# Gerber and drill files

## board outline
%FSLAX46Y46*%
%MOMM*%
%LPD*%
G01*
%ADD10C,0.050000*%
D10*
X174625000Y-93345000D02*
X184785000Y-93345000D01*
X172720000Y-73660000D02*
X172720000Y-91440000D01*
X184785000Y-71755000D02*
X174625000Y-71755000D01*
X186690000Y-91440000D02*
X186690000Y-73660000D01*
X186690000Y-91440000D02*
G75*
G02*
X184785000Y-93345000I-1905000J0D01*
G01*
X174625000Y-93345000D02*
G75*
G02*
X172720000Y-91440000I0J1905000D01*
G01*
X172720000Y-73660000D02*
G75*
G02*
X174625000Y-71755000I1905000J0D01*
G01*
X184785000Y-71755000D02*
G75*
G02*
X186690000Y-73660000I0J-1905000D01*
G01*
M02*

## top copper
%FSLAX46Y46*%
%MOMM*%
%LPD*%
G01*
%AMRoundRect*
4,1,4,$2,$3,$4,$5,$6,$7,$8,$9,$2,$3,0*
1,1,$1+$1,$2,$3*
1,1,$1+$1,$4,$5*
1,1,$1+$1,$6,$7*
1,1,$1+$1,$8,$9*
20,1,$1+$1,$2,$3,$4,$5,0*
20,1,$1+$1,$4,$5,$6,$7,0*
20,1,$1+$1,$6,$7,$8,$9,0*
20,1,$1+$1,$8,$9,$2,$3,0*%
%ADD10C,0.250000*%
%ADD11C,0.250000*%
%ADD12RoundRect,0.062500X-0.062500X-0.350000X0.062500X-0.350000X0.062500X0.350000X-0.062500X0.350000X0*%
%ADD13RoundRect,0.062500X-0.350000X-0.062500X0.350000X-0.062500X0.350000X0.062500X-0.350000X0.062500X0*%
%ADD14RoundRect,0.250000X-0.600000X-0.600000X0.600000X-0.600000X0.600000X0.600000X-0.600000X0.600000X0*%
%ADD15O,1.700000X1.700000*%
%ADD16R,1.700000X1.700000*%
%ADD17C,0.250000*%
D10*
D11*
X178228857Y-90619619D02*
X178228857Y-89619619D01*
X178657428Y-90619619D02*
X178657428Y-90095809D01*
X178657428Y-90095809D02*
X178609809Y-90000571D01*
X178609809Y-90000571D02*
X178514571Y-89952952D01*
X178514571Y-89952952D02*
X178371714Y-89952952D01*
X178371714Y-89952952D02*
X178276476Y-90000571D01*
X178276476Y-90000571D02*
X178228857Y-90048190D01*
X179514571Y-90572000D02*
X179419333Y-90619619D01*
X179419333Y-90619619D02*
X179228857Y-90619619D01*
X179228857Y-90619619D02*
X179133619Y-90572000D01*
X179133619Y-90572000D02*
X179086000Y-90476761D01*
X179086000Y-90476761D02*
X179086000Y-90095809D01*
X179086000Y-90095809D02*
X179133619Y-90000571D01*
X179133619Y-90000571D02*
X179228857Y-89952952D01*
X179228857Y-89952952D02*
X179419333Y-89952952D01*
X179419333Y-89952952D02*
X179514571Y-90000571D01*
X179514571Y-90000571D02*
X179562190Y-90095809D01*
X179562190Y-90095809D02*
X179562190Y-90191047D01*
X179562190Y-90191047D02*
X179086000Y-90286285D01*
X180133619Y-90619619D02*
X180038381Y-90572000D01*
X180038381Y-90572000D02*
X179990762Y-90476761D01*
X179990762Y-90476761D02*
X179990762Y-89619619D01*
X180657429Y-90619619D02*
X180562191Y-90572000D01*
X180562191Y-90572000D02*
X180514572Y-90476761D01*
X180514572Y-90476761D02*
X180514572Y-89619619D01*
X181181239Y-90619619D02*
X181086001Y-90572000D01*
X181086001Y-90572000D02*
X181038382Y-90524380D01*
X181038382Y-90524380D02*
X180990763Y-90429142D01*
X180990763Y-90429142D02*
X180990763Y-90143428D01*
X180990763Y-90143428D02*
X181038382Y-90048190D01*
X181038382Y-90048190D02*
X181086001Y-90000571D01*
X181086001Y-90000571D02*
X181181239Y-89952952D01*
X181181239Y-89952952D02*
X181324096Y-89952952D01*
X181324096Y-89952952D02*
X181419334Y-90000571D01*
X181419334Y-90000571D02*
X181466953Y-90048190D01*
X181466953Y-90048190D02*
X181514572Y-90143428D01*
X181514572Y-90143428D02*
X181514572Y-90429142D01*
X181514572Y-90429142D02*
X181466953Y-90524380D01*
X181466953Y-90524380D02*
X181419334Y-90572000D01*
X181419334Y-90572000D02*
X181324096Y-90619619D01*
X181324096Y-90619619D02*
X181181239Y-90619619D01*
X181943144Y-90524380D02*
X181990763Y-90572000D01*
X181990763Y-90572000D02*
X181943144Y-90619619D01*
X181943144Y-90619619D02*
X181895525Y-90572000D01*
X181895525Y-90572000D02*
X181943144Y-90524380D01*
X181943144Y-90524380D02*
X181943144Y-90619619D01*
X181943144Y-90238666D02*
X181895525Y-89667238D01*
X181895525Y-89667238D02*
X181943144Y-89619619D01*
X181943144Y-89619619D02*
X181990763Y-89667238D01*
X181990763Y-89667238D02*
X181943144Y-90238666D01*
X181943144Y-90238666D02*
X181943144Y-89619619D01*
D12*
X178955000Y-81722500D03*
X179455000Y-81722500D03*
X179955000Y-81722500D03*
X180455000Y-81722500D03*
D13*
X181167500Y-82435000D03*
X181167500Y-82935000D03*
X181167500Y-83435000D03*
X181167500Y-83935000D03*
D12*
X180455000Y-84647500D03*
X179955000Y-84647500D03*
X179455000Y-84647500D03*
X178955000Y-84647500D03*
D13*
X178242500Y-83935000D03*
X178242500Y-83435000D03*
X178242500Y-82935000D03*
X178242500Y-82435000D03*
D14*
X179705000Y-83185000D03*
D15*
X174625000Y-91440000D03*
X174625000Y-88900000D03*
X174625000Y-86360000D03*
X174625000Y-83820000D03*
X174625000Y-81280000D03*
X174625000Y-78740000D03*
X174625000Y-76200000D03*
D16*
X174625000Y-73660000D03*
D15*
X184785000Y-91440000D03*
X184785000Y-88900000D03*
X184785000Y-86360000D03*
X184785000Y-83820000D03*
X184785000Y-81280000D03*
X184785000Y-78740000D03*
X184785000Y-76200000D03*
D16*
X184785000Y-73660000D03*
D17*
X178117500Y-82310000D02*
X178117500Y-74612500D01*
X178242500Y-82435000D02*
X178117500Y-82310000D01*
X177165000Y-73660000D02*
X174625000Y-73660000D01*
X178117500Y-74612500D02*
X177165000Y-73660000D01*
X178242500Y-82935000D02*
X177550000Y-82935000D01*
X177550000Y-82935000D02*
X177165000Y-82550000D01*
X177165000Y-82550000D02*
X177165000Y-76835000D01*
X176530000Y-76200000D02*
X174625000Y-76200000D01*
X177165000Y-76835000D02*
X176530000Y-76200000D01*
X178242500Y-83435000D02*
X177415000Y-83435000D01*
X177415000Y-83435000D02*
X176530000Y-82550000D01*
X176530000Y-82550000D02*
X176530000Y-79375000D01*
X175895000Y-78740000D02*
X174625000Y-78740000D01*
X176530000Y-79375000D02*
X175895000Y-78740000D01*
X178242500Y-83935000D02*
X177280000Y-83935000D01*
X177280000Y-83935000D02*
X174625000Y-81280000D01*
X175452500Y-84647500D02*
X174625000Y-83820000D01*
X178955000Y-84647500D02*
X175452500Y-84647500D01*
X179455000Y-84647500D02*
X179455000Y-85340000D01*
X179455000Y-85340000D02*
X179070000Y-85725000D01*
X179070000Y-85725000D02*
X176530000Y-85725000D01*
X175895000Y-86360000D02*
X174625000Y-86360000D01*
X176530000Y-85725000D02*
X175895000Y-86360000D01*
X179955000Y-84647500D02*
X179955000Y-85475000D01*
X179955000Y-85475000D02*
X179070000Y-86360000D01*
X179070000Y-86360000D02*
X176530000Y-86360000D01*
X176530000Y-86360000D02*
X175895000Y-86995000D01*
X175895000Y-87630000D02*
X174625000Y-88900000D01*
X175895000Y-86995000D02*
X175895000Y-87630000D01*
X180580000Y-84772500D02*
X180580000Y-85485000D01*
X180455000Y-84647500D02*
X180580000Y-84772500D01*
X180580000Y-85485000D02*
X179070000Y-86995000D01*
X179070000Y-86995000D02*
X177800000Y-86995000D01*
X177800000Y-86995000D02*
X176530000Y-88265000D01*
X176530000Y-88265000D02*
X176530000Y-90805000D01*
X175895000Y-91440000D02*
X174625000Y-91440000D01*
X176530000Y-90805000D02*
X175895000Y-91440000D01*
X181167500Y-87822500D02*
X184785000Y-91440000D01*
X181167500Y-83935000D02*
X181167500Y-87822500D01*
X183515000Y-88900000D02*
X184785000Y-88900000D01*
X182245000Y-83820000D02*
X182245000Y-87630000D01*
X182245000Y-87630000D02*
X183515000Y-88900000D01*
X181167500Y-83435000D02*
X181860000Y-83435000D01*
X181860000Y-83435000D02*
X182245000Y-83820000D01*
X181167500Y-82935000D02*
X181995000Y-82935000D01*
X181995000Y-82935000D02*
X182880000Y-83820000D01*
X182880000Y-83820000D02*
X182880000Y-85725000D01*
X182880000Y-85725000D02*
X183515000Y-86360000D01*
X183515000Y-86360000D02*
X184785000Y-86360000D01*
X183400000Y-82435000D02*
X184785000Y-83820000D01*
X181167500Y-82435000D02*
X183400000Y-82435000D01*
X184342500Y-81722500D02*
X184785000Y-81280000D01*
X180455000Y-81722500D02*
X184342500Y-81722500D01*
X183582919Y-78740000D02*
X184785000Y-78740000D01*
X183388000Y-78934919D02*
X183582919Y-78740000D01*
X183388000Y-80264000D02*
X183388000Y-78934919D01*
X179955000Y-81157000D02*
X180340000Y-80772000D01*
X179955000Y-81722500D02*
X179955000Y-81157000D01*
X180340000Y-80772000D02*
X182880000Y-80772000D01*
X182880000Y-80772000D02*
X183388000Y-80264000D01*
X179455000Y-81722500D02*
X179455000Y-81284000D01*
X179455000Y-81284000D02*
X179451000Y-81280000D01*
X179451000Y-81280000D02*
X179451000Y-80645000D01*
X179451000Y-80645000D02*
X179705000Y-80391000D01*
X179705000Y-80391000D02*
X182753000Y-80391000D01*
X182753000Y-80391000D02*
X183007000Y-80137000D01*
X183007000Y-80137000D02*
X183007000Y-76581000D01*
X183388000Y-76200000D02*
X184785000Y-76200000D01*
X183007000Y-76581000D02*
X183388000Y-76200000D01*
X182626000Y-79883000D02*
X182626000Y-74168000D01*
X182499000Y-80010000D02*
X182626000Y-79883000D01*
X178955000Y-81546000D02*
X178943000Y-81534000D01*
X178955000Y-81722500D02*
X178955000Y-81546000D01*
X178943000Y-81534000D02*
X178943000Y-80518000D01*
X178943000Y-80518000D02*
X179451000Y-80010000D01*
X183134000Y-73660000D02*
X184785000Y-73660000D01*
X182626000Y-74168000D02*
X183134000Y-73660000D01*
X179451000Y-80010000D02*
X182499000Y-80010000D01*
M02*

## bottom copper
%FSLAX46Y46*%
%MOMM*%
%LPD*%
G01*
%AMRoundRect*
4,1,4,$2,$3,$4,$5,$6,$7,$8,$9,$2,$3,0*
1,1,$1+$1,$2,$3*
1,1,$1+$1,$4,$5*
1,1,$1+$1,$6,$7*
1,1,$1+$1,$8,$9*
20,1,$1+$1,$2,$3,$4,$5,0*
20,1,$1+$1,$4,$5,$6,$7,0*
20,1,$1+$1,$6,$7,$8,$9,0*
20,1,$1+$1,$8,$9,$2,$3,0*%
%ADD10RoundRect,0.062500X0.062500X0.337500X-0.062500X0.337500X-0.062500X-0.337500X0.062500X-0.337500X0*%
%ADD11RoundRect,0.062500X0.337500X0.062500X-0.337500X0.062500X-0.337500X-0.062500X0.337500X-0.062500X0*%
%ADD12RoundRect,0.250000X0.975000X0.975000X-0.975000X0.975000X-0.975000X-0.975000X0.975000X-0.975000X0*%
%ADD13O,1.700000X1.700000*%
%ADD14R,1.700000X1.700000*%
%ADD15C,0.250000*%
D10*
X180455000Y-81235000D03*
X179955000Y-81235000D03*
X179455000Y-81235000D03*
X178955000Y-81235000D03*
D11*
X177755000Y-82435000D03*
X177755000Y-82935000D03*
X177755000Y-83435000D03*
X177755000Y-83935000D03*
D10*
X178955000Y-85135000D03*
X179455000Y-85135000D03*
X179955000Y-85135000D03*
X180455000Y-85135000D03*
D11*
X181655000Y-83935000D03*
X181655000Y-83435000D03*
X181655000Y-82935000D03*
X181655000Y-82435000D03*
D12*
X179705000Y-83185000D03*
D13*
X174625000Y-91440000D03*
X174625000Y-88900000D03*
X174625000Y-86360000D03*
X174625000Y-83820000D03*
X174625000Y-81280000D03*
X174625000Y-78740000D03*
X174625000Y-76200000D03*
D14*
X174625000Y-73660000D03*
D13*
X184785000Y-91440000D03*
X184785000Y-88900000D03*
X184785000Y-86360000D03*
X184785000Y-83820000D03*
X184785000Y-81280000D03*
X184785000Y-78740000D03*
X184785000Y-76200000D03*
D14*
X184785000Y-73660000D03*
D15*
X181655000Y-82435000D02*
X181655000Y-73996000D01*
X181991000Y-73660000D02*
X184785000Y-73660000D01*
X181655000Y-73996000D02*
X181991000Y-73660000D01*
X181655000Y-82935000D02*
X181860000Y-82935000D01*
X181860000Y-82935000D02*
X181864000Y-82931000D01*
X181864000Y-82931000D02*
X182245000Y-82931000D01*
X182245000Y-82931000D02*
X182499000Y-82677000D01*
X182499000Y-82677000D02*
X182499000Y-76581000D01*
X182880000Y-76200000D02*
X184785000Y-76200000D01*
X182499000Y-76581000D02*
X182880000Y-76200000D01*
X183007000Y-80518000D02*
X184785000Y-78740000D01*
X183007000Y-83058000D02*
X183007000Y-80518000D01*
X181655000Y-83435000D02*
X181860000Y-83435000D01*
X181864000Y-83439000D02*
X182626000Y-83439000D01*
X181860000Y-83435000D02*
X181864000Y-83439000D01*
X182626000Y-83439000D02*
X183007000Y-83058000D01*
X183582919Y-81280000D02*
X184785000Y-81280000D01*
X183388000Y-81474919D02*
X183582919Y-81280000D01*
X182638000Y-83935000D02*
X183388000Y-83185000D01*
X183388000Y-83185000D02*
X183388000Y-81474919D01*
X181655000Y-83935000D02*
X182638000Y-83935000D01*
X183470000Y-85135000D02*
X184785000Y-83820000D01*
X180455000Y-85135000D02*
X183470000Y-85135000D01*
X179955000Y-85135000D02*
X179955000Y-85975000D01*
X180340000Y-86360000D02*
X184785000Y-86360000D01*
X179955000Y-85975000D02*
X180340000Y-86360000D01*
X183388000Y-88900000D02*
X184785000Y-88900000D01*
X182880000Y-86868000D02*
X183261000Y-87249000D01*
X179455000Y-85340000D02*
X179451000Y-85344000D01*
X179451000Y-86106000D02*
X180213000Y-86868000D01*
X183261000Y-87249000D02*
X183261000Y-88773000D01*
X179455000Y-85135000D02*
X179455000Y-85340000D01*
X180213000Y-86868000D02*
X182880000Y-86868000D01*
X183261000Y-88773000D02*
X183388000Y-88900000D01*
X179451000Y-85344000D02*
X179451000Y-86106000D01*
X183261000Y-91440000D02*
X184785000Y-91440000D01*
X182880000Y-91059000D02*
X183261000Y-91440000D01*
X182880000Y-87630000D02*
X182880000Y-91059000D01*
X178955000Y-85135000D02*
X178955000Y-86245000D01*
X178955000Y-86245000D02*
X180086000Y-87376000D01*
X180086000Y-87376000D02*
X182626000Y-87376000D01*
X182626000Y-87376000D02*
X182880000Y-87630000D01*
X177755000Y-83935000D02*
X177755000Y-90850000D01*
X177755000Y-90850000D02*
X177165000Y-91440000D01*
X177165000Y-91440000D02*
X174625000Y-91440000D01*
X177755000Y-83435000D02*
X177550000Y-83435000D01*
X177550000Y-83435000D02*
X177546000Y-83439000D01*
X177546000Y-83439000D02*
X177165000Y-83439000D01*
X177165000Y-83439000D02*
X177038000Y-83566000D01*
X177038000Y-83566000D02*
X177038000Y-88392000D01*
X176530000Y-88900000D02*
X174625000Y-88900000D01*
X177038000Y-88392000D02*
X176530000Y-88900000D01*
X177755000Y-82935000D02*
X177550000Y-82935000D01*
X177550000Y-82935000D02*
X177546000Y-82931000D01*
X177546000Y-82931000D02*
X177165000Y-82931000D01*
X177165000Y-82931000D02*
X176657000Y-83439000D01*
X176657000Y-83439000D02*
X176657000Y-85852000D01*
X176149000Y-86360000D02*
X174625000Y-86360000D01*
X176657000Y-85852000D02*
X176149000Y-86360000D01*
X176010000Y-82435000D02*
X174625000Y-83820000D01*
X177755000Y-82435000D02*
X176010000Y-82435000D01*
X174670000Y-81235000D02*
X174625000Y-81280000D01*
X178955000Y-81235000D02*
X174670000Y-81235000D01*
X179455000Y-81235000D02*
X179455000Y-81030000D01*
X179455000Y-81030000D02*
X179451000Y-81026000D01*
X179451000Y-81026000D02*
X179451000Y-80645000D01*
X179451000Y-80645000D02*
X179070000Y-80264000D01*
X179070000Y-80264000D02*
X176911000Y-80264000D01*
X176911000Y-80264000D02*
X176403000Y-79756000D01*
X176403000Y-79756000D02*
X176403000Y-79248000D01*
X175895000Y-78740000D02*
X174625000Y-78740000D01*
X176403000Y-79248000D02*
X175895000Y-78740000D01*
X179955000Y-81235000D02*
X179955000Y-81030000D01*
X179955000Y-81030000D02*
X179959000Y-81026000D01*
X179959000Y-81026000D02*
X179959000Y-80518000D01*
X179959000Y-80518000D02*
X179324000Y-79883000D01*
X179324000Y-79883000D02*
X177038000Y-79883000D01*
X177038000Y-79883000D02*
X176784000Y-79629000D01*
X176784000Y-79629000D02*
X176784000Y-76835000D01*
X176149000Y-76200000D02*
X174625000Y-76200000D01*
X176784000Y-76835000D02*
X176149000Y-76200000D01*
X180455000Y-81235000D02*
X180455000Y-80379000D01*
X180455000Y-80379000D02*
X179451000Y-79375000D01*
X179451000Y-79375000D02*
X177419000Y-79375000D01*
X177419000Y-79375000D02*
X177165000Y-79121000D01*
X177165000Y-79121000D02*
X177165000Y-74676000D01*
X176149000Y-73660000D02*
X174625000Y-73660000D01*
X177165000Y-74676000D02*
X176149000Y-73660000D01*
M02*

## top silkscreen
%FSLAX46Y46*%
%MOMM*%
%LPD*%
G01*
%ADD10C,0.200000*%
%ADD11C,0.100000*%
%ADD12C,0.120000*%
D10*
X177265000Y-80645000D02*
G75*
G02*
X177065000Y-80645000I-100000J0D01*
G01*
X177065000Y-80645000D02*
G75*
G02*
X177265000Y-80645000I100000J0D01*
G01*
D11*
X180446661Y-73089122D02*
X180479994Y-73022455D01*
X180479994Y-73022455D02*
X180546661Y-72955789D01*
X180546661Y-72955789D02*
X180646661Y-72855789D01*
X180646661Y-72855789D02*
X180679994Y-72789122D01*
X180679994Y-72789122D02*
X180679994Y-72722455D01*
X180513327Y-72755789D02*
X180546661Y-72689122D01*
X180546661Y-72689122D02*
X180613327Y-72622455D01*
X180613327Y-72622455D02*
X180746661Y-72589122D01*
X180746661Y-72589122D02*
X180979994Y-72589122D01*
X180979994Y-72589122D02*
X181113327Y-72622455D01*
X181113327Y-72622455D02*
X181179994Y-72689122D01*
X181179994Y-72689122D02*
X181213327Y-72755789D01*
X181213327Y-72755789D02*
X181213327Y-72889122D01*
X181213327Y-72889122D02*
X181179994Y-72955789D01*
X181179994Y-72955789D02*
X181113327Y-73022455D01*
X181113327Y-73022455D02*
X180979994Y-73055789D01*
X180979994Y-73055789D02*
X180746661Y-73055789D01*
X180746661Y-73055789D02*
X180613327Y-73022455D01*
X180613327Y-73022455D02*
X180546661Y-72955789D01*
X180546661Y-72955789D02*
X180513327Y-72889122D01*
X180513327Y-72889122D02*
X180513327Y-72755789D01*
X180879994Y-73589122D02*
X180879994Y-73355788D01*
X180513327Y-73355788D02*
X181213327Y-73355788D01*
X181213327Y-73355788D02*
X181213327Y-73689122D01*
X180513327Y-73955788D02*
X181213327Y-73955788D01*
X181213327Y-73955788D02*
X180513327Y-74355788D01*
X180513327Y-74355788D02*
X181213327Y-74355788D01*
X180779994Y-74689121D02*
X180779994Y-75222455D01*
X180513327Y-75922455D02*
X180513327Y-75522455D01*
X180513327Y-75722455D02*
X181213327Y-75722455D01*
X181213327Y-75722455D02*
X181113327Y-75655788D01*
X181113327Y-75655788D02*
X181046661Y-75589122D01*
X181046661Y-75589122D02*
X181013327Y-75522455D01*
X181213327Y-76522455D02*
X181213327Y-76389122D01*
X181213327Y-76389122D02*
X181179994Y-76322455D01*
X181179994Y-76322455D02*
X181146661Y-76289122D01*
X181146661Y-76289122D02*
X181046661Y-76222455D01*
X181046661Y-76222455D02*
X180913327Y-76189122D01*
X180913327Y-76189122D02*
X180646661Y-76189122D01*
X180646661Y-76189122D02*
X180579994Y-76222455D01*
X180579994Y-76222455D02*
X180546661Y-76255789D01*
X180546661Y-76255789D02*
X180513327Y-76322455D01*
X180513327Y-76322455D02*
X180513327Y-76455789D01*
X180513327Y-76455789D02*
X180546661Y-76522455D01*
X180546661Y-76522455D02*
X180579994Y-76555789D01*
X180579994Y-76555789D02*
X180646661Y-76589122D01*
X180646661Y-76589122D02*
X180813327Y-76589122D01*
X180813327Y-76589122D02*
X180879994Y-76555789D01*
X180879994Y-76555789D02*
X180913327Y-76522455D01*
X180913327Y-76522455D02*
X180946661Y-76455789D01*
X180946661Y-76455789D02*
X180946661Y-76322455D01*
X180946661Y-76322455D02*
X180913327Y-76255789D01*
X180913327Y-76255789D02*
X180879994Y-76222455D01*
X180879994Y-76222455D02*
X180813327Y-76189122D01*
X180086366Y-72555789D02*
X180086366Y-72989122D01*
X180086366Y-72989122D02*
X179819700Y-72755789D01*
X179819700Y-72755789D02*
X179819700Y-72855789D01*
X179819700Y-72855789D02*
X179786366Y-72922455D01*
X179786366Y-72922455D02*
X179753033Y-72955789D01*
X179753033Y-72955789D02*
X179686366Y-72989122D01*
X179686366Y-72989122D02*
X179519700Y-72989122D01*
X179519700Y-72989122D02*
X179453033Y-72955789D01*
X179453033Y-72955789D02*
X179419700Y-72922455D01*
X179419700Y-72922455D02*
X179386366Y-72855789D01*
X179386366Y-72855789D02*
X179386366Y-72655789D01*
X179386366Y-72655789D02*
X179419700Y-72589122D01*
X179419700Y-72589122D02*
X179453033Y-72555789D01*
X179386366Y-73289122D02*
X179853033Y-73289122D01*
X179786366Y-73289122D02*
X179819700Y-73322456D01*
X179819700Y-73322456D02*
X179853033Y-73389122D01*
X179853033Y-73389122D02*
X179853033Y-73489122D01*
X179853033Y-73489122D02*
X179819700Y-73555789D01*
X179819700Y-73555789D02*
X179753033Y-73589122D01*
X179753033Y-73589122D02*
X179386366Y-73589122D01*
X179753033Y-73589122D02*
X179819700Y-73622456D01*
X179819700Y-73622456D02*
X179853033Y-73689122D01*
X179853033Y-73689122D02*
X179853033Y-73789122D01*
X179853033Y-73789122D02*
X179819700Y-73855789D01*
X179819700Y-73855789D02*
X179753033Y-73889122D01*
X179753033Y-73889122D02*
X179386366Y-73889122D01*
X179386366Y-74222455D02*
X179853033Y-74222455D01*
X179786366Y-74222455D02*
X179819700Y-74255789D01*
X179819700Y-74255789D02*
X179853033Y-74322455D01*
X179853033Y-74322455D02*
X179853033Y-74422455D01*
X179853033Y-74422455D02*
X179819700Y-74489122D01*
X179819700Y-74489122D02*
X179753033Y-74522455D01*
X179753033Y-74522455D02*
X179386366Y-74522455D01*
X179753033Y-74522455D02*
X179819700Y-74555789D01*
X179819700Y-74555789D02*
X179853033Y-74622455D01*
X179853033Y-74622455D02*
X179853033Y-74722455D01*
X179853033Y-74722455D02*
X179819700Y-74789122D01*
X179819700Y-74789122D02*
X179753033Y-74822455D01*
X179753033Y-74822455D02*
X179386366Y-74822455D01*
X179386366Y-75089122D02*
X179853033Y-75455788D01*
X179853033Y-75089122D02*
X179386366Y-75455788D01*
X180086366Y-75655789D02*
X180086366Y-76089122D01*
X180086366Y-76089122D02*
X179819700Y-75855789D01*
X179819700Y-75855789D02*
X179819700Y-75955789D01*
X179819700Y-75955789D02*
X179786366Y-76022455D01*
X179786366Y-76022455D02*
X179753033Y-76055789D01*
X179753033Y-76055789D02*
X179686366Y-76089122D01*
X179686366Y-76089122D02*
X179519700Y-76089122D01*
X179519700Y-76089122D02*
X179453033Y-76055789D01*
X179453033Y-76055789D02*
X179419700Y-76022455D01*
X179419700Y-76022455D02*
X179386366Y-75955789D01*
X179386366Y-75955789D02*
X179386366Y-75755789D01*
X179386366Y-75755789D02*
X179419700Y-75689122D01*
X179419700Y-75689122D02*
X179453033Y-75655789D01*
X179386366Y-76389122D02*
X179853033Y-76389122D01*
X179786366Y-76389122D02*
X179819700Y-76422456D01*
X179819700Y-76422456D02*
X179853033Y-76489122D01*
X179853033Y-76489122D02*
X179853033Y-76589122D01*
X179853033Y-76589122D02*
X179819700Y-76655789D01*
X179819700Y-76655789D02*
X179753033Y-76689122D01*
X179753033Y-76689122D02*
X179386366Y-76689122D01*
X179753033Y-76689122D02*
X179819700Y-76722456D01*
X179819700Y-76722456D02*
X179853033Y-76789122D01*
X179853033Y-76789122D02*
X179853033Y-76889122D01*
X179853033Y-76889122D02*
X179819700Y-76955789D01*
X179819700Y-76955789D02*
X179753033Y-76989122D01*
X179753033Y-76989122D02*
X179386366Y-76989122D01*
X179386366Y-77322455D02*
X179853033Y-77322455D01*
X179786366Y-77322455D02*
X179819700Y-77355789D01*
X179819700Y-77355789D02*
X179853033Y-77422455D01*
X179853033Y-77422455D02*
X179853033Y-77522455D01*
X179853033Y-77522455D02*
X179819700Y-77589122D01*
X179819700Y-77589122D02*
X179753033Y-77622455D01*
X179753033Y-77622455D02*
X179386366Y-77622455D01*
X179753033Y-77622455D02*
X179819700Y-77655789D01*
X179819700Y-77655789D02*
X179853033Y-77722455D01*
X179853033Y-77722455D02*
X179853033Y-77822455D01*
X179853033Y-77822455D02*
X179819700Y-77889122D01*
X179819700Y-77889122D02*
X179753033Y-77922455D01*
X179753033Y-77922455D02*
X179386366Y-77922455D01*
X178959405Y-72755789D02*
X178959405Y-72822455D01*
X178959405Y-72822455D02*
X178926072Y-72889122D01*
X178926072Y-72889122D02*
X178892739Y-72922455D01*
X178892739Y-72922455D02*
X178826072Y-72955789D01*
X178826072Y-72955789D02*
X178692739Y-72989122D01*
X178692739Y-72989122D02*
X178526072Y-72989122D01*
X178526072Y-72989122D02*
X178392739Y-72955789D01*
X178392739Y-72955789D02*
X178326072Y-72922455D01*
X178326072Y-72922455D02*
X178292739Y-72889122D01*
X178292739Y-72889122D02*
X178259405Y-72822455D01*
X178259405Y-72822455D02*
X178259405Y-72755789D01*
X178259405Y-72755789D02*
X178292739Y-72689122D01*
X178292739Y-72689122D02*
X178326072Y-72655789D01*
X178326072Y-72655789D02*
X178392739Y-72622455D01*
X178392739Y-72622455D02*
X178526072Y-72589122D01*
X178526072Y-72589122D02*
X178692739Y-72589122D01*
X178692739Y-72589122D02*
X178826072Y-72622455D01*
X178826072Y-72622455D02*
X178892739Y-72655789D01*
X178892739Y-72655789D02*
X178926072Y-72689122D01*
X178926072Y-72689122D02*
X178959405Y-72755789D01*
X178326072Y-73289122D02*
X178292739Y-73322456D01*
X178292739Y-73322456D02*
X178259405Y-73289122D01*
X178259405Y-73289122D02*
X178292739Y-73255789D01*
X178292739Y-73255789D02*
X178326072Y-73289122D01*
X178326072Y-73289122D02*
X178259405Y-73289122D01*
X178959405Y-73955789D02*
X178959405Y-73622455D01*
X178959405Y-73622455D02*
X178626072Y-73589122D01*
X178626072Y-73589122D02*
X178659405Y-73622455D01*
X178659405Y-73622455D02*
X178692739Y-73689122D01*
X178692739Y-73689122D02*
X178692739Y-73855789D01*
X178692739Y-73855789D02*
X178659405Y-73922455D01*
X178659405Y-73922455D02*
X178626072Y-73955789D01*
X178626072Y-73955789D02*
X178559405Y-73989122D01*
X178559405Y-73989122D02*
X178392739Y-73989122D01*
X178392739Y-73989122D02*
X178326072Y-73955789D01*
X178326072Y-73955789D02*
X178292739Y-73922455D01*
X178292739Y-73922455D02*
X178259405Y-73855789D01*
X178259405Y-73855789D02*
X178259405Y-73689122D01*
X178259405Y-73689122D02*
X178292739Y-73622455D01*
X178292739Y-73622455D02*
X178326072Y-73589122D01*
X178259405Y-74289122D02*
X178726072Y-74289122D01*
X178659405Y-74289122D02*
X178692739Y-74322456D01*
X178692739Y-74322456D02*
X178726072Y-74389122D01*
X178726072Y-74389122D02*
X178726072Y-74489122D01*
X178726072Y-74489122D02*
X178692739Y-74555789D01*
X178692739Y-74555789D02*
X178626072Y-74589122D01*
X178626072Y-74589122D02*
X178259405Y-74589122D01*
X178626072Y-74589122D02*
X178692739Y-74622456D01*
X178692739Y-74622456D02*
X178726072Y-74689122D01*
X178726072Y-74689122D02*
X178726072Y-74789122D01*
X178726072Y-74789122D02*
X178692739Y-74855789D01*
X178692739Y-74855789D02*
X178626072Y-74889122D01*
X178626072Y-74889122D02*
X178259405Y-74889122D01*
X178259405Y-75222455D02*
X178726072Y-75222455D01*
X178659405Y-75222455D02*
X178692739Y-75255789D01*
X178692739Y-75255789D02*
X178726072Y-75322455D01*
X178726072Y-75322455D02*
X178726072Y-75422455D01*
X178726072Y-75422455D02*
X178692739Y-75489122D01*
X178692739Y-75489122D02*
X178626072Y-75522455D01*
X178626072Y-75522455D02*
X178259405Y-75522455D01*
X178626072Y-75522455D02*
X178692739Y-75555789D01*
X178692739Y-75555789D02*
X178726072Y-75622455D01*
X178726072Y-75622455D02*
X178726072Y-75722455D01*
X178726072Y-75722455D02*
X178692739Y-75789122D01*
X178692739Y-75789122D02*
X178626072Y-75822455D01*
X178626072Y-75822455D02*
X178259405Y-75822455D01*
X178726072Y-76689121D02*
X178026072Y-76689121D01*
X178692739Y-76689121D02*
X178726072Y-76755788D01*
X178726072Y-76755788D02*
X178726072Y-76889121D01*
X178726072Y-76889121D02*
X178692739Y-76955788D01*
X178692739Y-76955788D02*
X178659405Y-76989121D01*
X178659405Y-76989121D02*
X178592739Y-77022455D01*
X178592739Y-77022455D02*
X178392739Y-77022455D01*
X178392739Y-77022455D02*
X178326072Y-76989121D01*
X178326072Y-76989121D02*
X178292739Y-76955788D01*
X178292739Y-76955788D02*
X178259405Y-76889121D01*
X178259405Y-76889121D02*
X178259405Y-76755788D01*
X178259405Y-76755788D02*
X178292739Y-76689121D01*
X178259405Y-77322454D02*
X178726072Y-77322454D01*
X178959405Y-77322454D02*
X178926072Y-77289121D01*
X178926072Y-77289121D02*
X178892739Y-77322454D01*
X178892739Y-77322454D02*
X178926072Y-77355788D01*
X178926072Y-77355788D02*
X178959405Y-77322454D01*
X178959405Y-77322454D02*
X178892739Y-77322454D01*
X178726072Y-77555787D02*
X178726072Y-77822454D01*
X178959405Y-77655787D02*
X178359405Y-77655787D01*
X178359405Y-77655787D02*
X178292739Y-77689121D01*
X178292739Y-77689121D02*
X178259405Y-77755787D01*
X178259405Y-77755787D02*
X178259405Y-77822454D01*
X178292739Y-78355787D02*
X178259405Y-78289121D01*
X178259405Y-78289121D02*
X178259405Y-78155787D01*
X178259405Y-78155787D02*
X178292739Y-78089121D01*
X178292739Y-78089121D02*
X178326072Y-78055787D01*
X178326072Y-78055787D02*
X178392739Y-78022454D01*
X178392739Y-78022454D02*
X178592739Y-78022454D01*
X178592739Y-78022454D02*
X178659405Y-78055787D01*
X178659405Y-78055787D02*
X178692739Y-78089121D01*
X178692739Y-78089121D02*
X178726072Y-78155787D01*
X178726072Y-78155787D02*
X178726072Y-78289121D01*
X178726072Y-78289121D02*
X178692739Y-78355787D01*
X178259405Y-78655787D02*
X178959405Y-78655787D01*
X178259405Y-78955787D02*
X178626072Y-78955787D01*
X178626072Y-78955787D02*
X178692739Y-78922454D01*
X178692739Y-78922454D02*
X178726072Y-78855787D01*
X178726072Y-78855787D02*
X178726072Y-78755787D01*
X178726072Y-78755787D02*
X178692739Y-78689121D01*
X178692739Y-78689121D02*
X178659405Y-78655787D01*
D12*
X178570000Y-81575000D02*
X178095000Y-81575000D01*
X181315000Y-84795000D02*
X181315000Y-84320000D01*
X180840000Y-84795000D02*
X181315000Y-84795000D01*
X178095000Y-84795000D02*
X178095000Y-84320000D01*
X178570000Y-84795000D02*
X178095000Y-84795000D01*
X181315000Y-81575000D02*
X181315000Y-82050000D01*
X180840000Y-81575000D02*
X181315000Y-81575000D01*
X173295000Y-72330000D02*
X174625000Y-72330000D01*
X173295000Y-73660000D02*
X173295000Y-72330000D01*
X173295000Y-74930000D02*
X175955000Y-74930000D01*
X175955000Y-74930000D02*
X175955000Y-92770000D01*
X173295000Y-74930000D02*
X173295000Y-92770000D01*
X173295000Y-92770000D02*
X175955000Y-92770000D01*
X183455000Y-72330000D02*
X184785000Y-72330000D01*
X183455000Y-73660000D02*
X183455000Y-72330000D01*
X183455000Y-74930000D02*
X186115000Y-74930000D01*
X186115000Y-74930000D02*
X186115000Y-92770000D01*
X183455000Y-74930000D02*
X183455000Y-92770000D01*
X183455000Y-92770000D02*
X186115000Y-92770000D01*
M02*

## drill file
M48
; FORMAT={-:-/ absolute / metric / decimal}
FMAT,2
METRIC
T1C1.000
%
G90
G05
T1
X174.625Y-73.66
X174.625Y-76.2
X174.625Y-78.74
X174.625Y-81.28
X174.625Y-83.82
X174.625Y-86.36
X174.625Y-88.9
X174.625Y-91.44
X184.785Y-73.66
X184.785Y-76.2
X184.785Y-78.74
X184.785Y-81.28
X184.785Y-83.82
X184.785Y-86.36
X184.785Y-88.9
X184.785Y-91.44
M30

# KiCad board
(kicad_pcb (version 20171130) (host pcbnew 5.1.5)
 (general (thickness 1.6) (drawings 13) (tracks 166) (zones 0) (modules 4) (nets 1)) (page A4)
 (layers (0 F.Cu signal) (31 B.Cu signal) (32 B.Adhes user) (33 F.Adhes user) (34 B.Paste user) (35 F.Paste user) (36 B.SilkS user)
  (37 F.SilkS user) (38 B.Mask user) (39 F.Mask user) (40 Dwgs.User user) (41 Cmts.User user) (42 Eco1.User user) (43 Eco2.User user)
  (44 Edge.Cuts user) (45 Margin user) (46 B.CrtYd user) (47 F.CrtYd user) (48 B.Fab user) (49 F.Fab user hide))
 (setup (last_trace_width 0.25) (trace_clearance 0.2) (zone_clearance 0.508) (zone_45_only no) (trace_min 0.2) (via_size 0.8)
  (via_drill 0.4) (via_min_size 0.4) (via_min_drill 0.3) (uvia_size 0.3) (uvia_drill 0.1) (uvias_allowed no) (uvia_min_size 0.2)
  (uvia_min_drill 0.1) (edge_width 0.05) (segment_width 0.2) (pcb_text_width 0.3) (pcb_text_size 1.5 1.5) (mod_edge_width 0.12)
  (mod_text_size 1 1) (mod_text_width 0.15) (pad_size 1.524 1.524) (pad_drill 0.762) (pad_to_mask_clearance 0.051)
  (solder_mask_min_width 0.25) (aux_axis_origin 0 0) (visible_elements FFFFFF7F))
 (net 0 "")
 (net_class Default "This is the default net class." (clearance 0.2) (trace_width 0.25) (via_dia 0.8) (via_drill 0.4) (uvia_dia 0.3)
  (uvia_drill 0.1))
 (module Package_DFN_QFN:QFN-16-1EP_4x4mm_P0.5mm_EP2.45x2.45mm (layer B.Cu) (at 179.705 83.185 180)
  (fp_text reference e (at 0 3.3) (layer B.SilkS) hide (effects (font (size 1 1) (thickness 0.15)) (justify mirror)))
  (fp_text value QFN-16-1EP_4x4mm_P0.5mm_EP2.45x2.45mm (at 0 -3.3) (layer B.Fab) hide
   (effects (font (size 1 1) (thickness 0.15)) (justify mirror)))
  (pad 16 smd roundrect (at -0.75 1.95 180) (size 0.25 0.8) (layers B.Cu B.Paste B.Mask) (roundrect_rratio 0.25))
  (pad 15 smd roundrect (at -0.25 1.95 180) (size 0.25 0.8) (layers B.Cu B.Paste B.Mask) (roundrect_rratio 0.25))
  (pad 14 smd roundrect (at 0.25 1.95 180) (size 0.25 0.8) (layers B.Cu B.Paste B.Mask) (roundrect_rratio 0.25))
  (pad 13 smd roundrect (at 0.75 1.95 180) (size 0.25 0.8) (layers B.Cu B.Paste B.Mask) (roundrect_rratio 0.25))
  (pad 12 smd roundrect (at 1.95 0.75 180) (size 0.8 0.25) (layers B.Cu B.Paste B.Mask) (roundrect_rratio 0.25))
  (pad 11 smd roundrect (at 1.95 0.25 180) (size 0.8 0.25) (layers B.Cu B.Paste B.Mask) (roundrect_rratio 0.25))
  (pad 10 smd roundrect (at 1.95 -0.25 180) (size 0.8 0.25) (layers B.Cu B.Paste B.Mask) (roundrect_rratio 0.25))
  (pad 9 smd roundrect (at 1.95 -0.75 180) (size 0.8 0.25) (layers B.Cu B.Paste B.Mask) (roundrect_rratio 0.25))
  (pad 8 smd roundrect (at 0.75 -1.95 180) (size 0.25 0.8) (layers B.Cu B.Paste B.Mask) (roundrect_rratio 0.25))
  (pad 7 smd roundrect (at 0.25 -1.95 180) (size 0.25 0.8) (layers B.Cu B.Paste B.Mask) (roundrect_rratio 0.25))
  (pad 6 smd roundrect (at -0.25 -1.95 180) (size 0.25 0.8) (layers B.Cu B.Paste B.Mask) (roundrect_rratio 0.25))
  (pad 5 smd roundrect (at -0.75 -1.95 180) (size 0.25 0.8) (layers B.Cu B.Paste B.Mask) (roundrect_rratio 0.25))
  (pad 4 smd roundrect (at -1.95 -0.75 180) (size 0.8 0.25) (layers B.Cu B.Paste B.Mask) (roundrect_rratio 0.25))
  (pad 3 smd roundrect (at -1.95 -0.25 180) (size 0.8 0.25) (layers B.Cu B.Paste B.Mask) (roundrect_rratio 0.25))
  (pad 2 smd roundrect (at -1.95 0.25 180) (size 0.8 0.25) (layers B.Cu B.Paste B.Mask) (roundrect_rratio 0.25))
  (pad 1 smd roundrect (at -1.95 0.75 180) (size 0.8 0.25) (layers B.Cu B.Paste B.Mask) (roundrect_rratio 0.25))
  (pad "" smd roundrect (at 0.61 -0.61 180) (size 0.99 0.99) (layers B.Paste) (roundrect_rratio 0.25))
  (pad "" smd roundrect (at 0.61 0.61 180) (size 0.99 0.99) (layers B.Paste) (roundrect_rratio 0.25))
  (pad "" smd roundrect (at -0.61 -0.61 180) (size 0.99 0.99) (layers B.Paste) (roundrect_rratio 0.25))
  (pad "" smd roundrect (at -0.61 0.61 180) (size 0.99 0.99) (layers B.Paste) (roundrect_rratio 0.25))
  (pad 17 smd roundrect (at 0 0 180) (size 2.45 2.45) (layers B.Cu B.Mask) (roundrect_rratio 0.102041)))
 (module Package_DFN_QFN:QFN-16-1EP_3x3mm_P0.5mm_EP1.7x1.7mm (layer F.Cu) (at 179.705 83.185)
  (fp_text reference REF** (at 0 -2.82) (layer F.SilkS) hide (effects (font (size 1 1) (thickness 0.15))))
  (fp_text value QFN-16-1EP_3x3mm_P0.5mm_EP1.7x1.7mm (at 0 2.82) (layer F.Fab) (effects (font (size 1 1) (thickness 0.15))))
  (fp_line (start -1.135 -1.61) (end -1.61 -1.61) (layer F.SilkS) (width 0.12))
  (fp_line (start 1.61 1.61) (end 1.61 1.135) (layer F.SilkS) (width 0.12))
  (fp_line (start 1.135 1.61) (end 1.61 1.61) (layer F.SilkS) (width 0.12))
  (fp_line (start -1.61 1.61) (end -1.61 1.135) (layer F.SilkS) (width 0.12))
  (fp_line (start -1.135 1.61) (end -1.61 1.61) (layer F.SilkS) (width 0.12))
  (fp_line (start 1.61 -1.61) (end 1.61 -1.135) (layer F.SilkS) (width 0.12))
  (fp_line (start 1.135 -1.61) (end 1.61 -1.61) (layer F.SilkS) (width 0.12))
  (pad 16 smd roundrect (at -0.75 -1.4625) (size 0.25 0.825) (layers F.Cu F.Paste F.Mask) (roundrect_rratio 0.25))
  (pad 15 smd roundrect (at -0.25 -1.4625) (size 0.25 0.825) (layers F.Cu F.Paste F.Mask) (roundrect_rratio 0.25))
  (pad 14 smd roundrect (at 0.25 -1.4625) (size 0.25 0.825) (layers F.Cu F.Paste F.Mask) (roundrect_rratio 0.25))
  (pad 13 smd roundrect (at 0.75 -1.4625) (size 0.25 0.825) (layers F.Cu F.Paste F.Mask) (roundrect_rratio 0.25))
  (pad 12 smd roundrect (at 1.4625 -0.75) (size 0.825 0.25) (layers F.Cu F.Paste F.Mask) (roundrect_rratio 0.25))
  (pad 11 smd roundrect (at 1.4625 -0.25) (size 0.825 0.25) (layers F.Cu F.Paste F.Mask) (roundrect_rratio 0.25))
  (pad 10 smd roundrect (at 1.4625 0.25) (size 0.825 0.25) (layers F.Cu F.Paste F.Mask) (roundrect_rratio 0.25))
  (pad 9 smd roundrect (at 1.4625 0.75) (size 0.825 0.25) (layers F.Cu F.Paste F.Mask) (roundrect_rratio 0.25))
  (pad 8 smd roundrect (at 0.75 1.4625) (size 0.25 0.825) (layers F.Cu F.Paste F.Mask) (roundrect_rratio 0.25))
  (pad 7 smd roundrect (at 0.25 1.4625) (size 0.25 0.825) (layers F.Cu F.Paste F.Mask) (roundrect_rratio 0.25))
  (pad 6 smd roundrect (at -0.25 1.4625) (size 0.25 0.825) (layers F.Cu F.Paste F.Mask) (roundrect_rratio 0.25))
  (pad 5 smd roundrect (at -0.75 1.4625) (size 0.25 0.825) (layers F.Cu F.Paste F.Mask) (roundrect_rratio 0.25))
  (pad 4 smd roundrect (at -1.4625 0.75) (size 0.825 0.25) (layers F.Cu F.Paste F.Mask) (roundrect_rratio 0.25))
  (pad 3 smd roundrect (at -1.4625 0.25) (size 0.825 0.25) (layers F.Cu F.Paste F.Mask) (roundrect_rratio 0.25))
  (pad 2 smd roundrect (at -1.4625 -0.25) (size 0.825 0.25) (layers F.Cu F.Paste F.Mask) (roundrect_rratio 0.25))
  (pad 1 smd roundrect (at -1.4625 -0.75) (size 0.825 0.25) (layers F.Cu F.Paste F.Mask) (roundrect_rratio 0.25))
  (pad "" smd roundrect (at 0.425 0.425) (size 0.69 0.69) (layers F.Paste) (roundrect_rratio 0.25))
  (pad "" smd roundrect (at 0.425 -0.425) (size 0.69 0.69) (layers F.Paste) (roundrect_rratio 0.25))
  (pad "" smd roundrect (at -0.425 0.425) (size 0.69 0.69) (layers F.Paste) (roundrect_rratio 0.25))
  (pad "" smd roundrect (at -0.425 -0.425) (size 0.69 0.69) (layers F.Paste) (roundrect_rratio 0.25))
  (pad 17 smd roundrect (at 0 0) (size 1.7 1.7) (layers F.Cu F.Mask) (roundrect_rratio 0.147059)))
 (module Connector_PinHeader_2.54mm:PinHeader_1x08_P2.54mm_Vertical (layer F.Cu) (at 174.625 73.66)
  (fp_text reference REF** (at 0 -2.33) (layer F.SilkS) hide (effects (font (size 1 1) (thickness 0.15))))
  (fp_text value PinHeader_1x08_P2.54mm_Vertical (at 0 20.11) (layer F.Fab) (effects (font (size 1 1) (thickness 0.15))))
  (fp_line (start -1.33 -1.33) (end 0 -1.33) (layer F.SilkS) (width 0.12))
  (fp_line (start -1.33 0) (end -1.33 -1.33) (layer F.SilkS) (width 0.12))
  (fp_line (start -1.33 1.27) (end 1.33 1.27) (layer F.SilkS) (width 0.12))
  (fp_line (start 1.33 1.27) (end 1.33 19.11) (layer F.SilkS) (width 0.12))
  (fp_line (start -1.33 1.27) (end -1.33 19.11) (layer F.SilkS) (width 0.12))
  (fp_line (start -1.33 19.11) (end 1.33 19.11) (layer F.SilkS) (width 0.12))
  (pad 8 thru_hole oval (at 0 17.78) (size 1.7 1.7) (drill 1) (layers *.Cu *.Mask))
  (pad 7 thru_hole oval (at 0 15.24) (size 1.7 1.7) (drill 1) (layers *.Cu *.Mask))
  (pad 6 thru_hole oval (at 0 12.7) (size 1.7 1.7) (drill 1) (layers *.Cu *.Mask))
  (pad 5 thru_hole oval (at 0 10.16) (size 1.7 1.7) (drill 1) (layers *.Cu *.Mask))
  (pad 4 thru_hole oval (at 0 7.62) (size 1.7 1.7) (drill 1) (layers *.Cu *.Mask))
  (pad 3 thru_hole oval (at 0 5.08) (size 1.7 1.7) (drill 1) (layers *.Cu *.Mask))
  (pad 2 thru_hole oval (at 0 2.54) (size 1.7 1.7) (drill 1) (layers *.Cu *.Mask))
  (pad 1 thru_hole rect (at 0 0) (size 1.7 1.7) (drill 1) (layers *.Cu *.Mask)))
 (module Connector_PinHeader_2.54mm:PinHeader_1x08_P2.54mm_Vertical (layer F.Cu) (at 184.785 73.66)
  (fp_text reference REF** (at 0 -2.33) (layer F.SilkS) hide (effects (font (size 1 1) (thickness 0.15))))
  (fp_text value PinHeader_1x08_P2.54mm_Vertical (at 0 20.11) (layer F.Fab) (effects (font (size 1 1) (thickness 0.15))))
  (fp_line (start -1.33 -1.33) (end 0 -1.33) (layer F.SilkS) (width 0.12))
  (fp_line (start -1.33 0) (end -1.33 -1.33) (layer F.SilkS) (width 0.12))
  (fp_line (start -1.33 1.27) (end 1.33 1.27) (layer F.SilkS) (width 0.12))
  (fp_line (start 1.33 1.27) (end 1.33 19.11) (layer F.SilkS) (width 0.12))
  (fp_line (start -1.33 1.27) (end -1.33 19.11) (layer F.SilkS) (width 0.12))
  (fp_line (start -1.33 19.11) (end 1.33 19.11) (layer F.SilkS) (width 0.12))
  (pad 8 thru_hole oval (at 0 17.78) (size 1.7 1.7) (drill 1) (layers *.Cu *.Mask))
  (pad 7 thru_hole oval (at 0 15.24) (size 1.7 1.7) (drill 1) (layers *.Cu *.Mask))
  (pad 6 thru_hole oval (at 0 12.7) (size 1.7 1.7) (drill 1) (layers *.Cu *.Mask))
  (pad 5 thru_hole oval (at 0 10.16) (size 1.7 1.7) (drill 1) (layers *.Cu *.Mask))
  (pad 4 thru_hole oval (at 0 7.62) (size 1.7 1.7) (drill 1) (layers *.Cu *.Mask))
  (pad 3 thru_hole oval (at 0 5.08) (size 1.7 1.7) (drill 1) (layers *.Cu *.Mask))
  (pad 2 thru_hole oval (at 0 2.54) (size 1.7 1.7) (drill 1) (layers *.Cu *.Mask))
  (pad 1 thru_hole rect (at 0 0) (size 1.7 1.7) (drill 1) (layers *.Cu *.Mask)))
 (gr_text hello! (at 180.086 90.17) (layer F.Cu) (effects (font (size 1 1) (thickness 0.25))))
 (gr_circle (center 177.165 80.645) (end 177.265 80.645) (layer F.SilkS) (width 0.2))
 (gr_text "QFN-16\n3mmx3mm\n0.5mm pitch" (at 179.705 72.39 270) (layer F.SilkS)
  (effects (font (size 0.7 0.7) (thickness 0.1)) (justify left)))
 (gr_line (start 174.625 93.345) (end 184.785 93.345) (layer Edge.Cuts) (width 0.05))
 (gr_line (start 172.72 73.66) (end 172.72 91.44) (layer Edge.Cuts) (width 0.05))
 (gr_line (start 184.785 71.755) (end 174.625 71.755) (layer Edge.Cuts) (width 0.05))
 (gr_line (start 186.69 91.44) (end 186.69 73.66) (layer Edge.Cuts) (width 0.05))
 (gr_arc (start 184.785 91.44) (end 184.785 93.345) (angle -90) (layer Edge.Cuts) (width 0.05))
 (gr_arc (start 174.625 91.44) (end 172.72 91.44) (angle -90) (layer Edge.Cuts) (width 0.05))
 (gr_arc (start 174.625 73.66) (end 174.625 71.755) (angle -90) (layer Edge.Cuts) (width 0.05))
 (gr_arc (start 184.785 73.66) (end 186.69 73.66) (angle -90) (layer Edge.Cuts) (width 0.05))
 (segment (start 178.1175 82.31) (end 178.1175 74.6125) (width 0.25) (layer F.Cu) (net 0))
 (segment (start 178.2425 82.435) (end 178.1175 82.31) (width 0.25) (layer F.Cu) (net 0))
 (segment (start 177.165 73.66) (end 174.625 73.66) (width 0.25) (layer F.Cu) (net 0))
 (segment (start 178.1175 74.6125) (end 177.165 73.66) (width 0.25) (layer F.Cu) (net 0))
 (segment (start 178.2425 82.935) (end 177.55 82.935) (width 0.25) (layer F.Cu) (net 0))
 (segment (start 177.55 82.935) (end 177.165 82.55) (width 0.25) (layer F.Cu) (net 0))
 (segment (start 177.165 82.55) (end 177.165 76.835) (width 0.25) (layer F.Cu) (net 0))
 (segment (start 176.53 76.2) (end 174.625 76.2) (width 0.25) (layer F.Cu) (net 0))
 (segment (start 177.165 76.835) (end 176.53 76.2) (width 0.25) (layer F.Cu) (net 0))
 (segment (start 178.2425 83.435) (end 177.415 83.435) (width 0.25) (layer F.Cu) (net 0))
 (segment (start 177.415 83.435) (end 176.53 82.55) (width 0.25) (layer F.Cu) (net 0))
 (segment (start 176.53 82.55) (end 176.53 79.375) (width 0.25) (layer F.Cu) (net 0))
 (segment (start 175.895 78.74) (end 174.625 78.74) (width 0.25) (layer F.Cu) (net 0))
 (segment (start 176.53 79.375) (end 175.895 78.74) (width 0.25) (layer F.Cu) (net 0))
 (segment (start 178.2425 83.935) (end 177.28 83.935) (width 0.25) (layer F.Cu) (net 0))
 (segment (start 177.28 83.935) (end 174.625 81.28) (width 0.25) (layer F.Cu) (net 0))
 (segment (start 175.4525 84.6475) (end 174.625 83.82) (width 0.25) (layer F.Cu) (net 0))
 (segment (start 178.955 84.6475) (end 175.4525 84.6475) (width 0.25) (layer F.Cu) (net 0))
 (segment (start 179.455 84.6475) (end 179.455 85.34) (width 0.25) (layer F.Cu) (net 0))
 (segment (start 179.455 85.34) (end 179.07 85.725) (width 0.25) (layer F.Cu) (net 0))
 (segment (start 179.07 85.725) (end 176.53 85.725) (width 0.25) (layer F.Cu) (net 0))
 (segment (start 175.895 86.36) (end 174.625 86.36) (width 0.25) (layer F.Cu) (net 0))
 (segment (start 176.53 85.725) (end 175.895 86.36) (width 0.25) (layer F.Cu) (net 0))
 (segment (start 179.955 84.6475) (end 179.955 85.475) (width 0.25) (layer F.Cu) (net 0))
 (segment (start 179.955 85.475) (end 179.07 86.36) (width 0.25) (layer F.Cu) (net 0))
 (segment (start 179.07 86.36) (end 176.53 86.36) (width 0.25) (layer F.Cu) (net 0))
 (segment (start 176.53 86.36) (end 175.895 86.995) (width 0.25) (layer F.Cu) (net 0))
 (segment (start 175.895 87.63) (end 174.625 88.9) (width 0.25) (layer F.Cu) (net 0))
 (segment (start 175.895 86.995) (end 175.895 87.63) (width 0.25) (layer F.Cu) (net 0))
 (segment (start 180.58 84.7725) (end 180.58 85.485) (width 0.25) (layer F.Cu) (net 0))
 (segment (start 180.455 84.6475) (end 180.58 84.7725) (width 0.25) (layer F.Cu) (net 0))
 (segment (start 180.58 85.485) (end 179.07 86.995) (width 0.25) (layer F.Cu) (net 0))
 (segment (start 179.07 86.995) (end 177.8 86.995) (width 0.25) (layer F.Cu) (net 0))
 (segment (start 177.8 86.995) (end 176.53 88.265) (width 0.25) (layer F.Cu) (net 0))
 (segment (start 176.53 88.265) (end 176.53 90.805) (width 0.25) (layer F.Cu) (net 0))
 (segment (start 175.895 91.44) (end 174.625 91.44) (width 0.25) (layer F.Cu) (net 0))
 (segment (start 176.53 90.805) (end 175.895 91.44) (width 0.25) (layer F.Cu) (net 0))
 (segment (start 181.1675 87.8225) (end 184.785 91.44) (width 0.25) (layer F.Cu) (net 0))
 (segment (start 181.1675 83.935) (end 181.1675 87.8225) (width 0.25) (layer F.Cu) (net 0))
 (segment (start 183.515 88.9) (end 184.785 88.9) (width 0.25) (layer F.Cu) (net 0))
 (segment (start 182.245 83.82) (end 182.245 87.63) (width 0.25) (layer F.Cu) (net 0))
 (segment (start 182.245 87.63) (end 183.515 88.9) (width 0.25) (layer F.Cu) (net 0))
 (segment (start 181.1675 83.435) (end 181.86 83.435) (width 0.25) (layer F.Cu) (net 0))
 (segment (start 181.86 83.435) (end 182.245 83.82) (width 0.25) (layer F.Cu) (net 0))
 (segment (start 181.1675 82.935) (end 181.995 82.935) (width 0.25) (layer F.Cu) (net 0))
 (segment (start 181.995 82.935) (end 182.88 83.82) (width 0.25) (layer F.Cu) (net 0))
 (segment (start 182.88 83.82) (end 182.88 85.725) (width 0.25) (layer F.Cu) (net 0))
 (segment (start 182.88 85.725) (end 183.515 86.36) (width 0.25) (layer F.Cu) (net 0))
 (segment (start 183.515 86.36) (end 184.785 86.36) (width 0.25) (layer F.Cu) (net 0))
 (segment (start 183.4 82.435) (end 184.785 83.82) (width 0.25) (layer F.Cu) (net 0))
 (segment (start 181.1675 82.435) (end 183.4 82.435) (width 0.25) (layer F.Cu) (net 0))
 (segment (start 184.3425 81.7225) (end 184.785 81.28) (width 0.25) (layer F.Cu) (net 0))
 (segment (start 180.455 81.7225) (end 184.3425 81.7225) (width 0.25) (layer F.Cu) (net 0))
 (segment (start 183.582919 78.74) (end 184.785 78.74) (width 0.25) (layer F.Cu) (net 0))
 (segment (start 183.388 78.934919) (end 183.582919 78.74) (width 0.25) (layer F.Cu) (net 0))
 (segment (start 183.388 80.264) (end 183.388 78.934919) (width 0.25) (layer F.Cu) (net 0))
 (segment (start 179.955 81.157) (end 180.34 80.772) (width 0.25) (layer F.Cu) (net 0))
 (segment (start 179.955 81.7225) (end 179.955 81.157) (width 0.25) (layer F.Cu) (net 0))
 (segment (start 180.34 80.772) (end 182.88 80.772) (width 0.25) (layer F.Cu) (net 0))
 (segment (start 182.88 80.772) (end 183.388 80.264) (width 0.25) (layer F.Cu) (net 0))
 (segment (start 179.455 81.7225) (end 179.455 81.284) (width 0.25) (layer F.Cu) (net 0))
 (segment (start 179.455 81.284) (end 179.451 81.28) (width 0.25) (layer F.Cu) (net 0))
 (segment (start 179.451 81.28) (end 179.451 80.645) (width 0.25) (layer F.Cu) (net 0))
 (segment (start 179.451 80.645) (end 179.705 80.391) (width 0.25) (layer F.Cu) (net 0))
 (segment (start 179.705 80.391) (end 182.753 80.391) (width 0.25) (layer F.Cu) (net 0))
 (segment (start 182.753 80.391) (end 183.007 80.137) (width 0.25) (layer F.Cu) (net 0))
 (segment (start 183.007 80.137) (end 183.007 76.581) (width 0.25) (layer F.Cu) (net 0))
 (segment (start 183.388 76.2) (end 184.785 76.2) (width 0.25) (layer F.Cu) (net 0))
 (segment (start 183.007 76.581) (end 183.388 76.2) (width 0.25) (layer F.Cu) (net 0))
 (segment (start 182.626 79.883) (end 182.626 74.168) (width 0.25) (layer F.Cu) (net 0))
 (segment (start 182.499 80.01) (end 182.626 79.883) (width 0.25) (layer F.Cu) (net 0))
 (segment (start 178.955 81.546) (end 178.943 81.534) (width 0.25) (layer F.Cu) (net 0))
 (segment (start 178.955 81.7225) (end 178.955 81.546) (width 0.25) (layer F.Cu) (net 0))
 (segment (start 178.943 81.534) (end 178.943 80.518) (width 0.25) (layer F.Cu) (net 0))
 (segment (start 178.943 80.518) (end 179.451 80.01) (width 0.25) (layer F.Cu) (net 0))
 (segment (start 183.134 73.66) (end 184.785 73.66) (width 0.25) (layer F.Cu) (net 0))
 (segment (start 182.626 74.168) (end 183.134 73.66) (width 0.25) (layer F.Cu) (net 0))
 (segment (start 179.451 80.01) (end 182.499 80.01) (width 0.25) (layer F.Cu) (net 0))
 (segment (start 181.655 82.435) (end 181.655 73.996) (width 0.25) (layer B.Cu) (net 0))
 (segment (start 181.991 73.66) (end 184.785 73.66) (width 0.25) (layer B.Cu) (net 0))
 (segment (start 181.655 73.996) (end 181.991 73.66) (width 0.25) (layer B.Cu) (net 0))
 (segment (start 181.655 82.935) (end 181.86 82.935) (width 0.25) (layer B.Cu) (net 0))
 (segment (start 181.86 82.935) (end 181.864 82.931) (width 0.25) (layer B.Cu) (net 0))
 (segment (start 181.864 82.931) (end 182.245 82.931) (width 0.25) (layer B.Cu) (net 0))
 (segment (start 182.245 82.931) (end 182.499 82.677) (width 0.25) (layer B.Cu) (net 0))
 (segment (start 182.499 82.677) (end 182.499 76.581) (width 0.25) (layer B.Cu) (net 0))
 (segment (start 182.88 76.2) (end 184.785 76.2) (width 0.25) (layer B.Cu) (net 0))
 (segment (start 182.499 76.581) (end 182.88 76.2) (width 0.25) (layer B.Cu) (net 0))
 (segment (start 183.007 80.518) (end 184.785 78.74) (width 0.25) (layer B.Cu) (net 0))
 (segment (start 183.007 83.058) (end 183.007 80.518) (width 0.25) (layer B.Cu) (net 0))
 (segment (start 181.655 83.435) (end 181.86 83.435) (width 0.25) (layer B.Cu) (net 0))
 (segment (start 181.864 83.439) (end 182.626 83.439) (width 0.25) (layer B.Cu) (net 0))
 (segment (start 181.86 83.435) (end 181.864 83.439) (width 0.25) (layer B.Cu) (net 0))
 (segment (start 182.626 83.439) (end 183.007 83.058) (width 0.25) (layer B.Cu) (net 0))
 (segment (start 183.582919 81.28) (end 184.785 81.28) (width 0.25) (layer B.Cu) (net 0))
 (segment (start 183.388 81.474919) (end 183.582919 81.28) (width 0.25) (layer B.Cu) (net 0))
 (segment (start 182.638 83.935) (end 183.388 83.185) (width 0.25) (layer B.Cu) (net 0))
 (segment (start 183.388 83.185) (end 183.388 81.474919) (width 0.25) (layer B.Cu) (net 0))
 (segment (start 181.655 83.935) (end 182.638 83.935) (width 0.25) (layer B.Cu) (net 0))
 (segment (start 183.47 85.135) (end 184.785 83.82) (width 0.25) (layer B.Cu) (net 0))
 (segment (start 180.455 85.135) (end 183.47 85.135) (width 0.25) (layer B.Cu) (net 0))
 (segment (start 179.955 85.135) (end 179.955 85.975) (width 0.25) (layer B.Cu) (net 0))
 (segment (start 180.34 86.36) (end 184.785 86.36) (width 0.25) (layer B.Cu) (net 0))
 (segment (start 179.955 85.975) (end 180.34 86.36) (width 0.25) (layer B.Cu) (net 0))
 (segment (start 183.388 88.9) (end 184.785 88.9) (width 0.25) (layer B.Cu) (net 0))
 (segment (start 182.88 86.868) (end 183.261 87.249) (width 0.25) (layer B.Cu) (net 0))
 (segment (start 179.455 85.34) (end 179.451 85.344) (width 0.25) (layer B.Cu) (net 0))
 (segment (start 179.451 86.106) (end 180.213 86.868) (width 0.25) (layer B.Cu) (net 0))
 (segment (start 183.261 87.249) (end 183.261 88.773) (width 0.25) (layer B.Cu) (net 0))
 (segment (start 179.455 85.135) (end 179.455 85.34) (width 0.25) (layer B.Cu) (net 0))
 (segment (start 180.213 86.868) (end 182.88 86.868) (width 0.25) (layer B.Cu) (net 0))
 (segment (start 183.261 88.773) (end 183.388 88.9) (width 0.25) (layer B.Cu) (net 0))
 (segment (start 179.451 85.344) (end 179.451 86.106) (width 0.25) (layer B.Cu) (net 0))
 (segment (start 183.261 91.44) (end 184.785 91.44) (width 0.25) (layer B.Cu) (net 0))
 (segment (start 182.88 91.059) (end 183.261 91.44) (width 0.25) (layer B.Cu) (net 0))
 (segment (start 182.88 87.63) (end 182.88 91.059) (width 0.25) (layer B.Cu) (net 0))
 (segment (start 178.955 85.135) (end 178.955 86.245) (width 0.25) (layer B.Cu) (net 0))
 (segment (start 178.955 86.245) (end 180.086 87.376) (width 0.25) (layer B.Cu) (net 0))
 (segment (start 180.086 87.376) (end 182.626 87.376) (width 0.25) (layer B.Cu) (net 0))
 (segment (start 182.626 87.376) (end 182.88 87.63) (width 0.25) (layer B.Cu) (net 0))
 (segment (start 177.755 83.935) (end 177.755 90.85) (width 0.25) (layer B.Cu) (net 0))
 (segment (start 177.755 90.85) (end 177.165 91.44) (width 0.25) (layer B.Cu) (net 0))
 (segment (start 177.165 91.44) (end 174.625 91.44) (width 0.25) (layer B.Cu) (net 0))
 (segment (start 177.755 83.435) (end 177.55 83.435) (width 0.25) (layer B.Cu) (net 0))
 (segment (start 177.55 83.435) (end 177.546 83.439) (width 0.25) (layer B.Cu) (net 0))
 (segment (start 177.546 83.439) (end 177.165 83.439) (width 0.25) (layer B.Cu) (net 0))
 (segment (start 177.165 83.439) (end 177.038 83.566) (width 0.25) (layer B.Cu) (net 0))
 (segment (start 177.038 83.566) (end 177.038 88.392) (width 0.25) (layer B.Cu) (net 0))
 (segment (start 176.53 88.9) (end 174.625 88.9) (width 0.25) (layer B.Cu) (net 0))
 (segment (start 177.038 88.392) (end 176.53 88.9) (width 0.25) (layer B.Cu) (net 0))
 (segment (start 177.755 82.935) (end 177.55 82.935) (width 0.25) (layer B.Cu) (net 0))
 (segment (start 177.55 82.935) (end 177.546 82.931) (width 0.25) (layer B.Cu) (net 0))
 (segment (start 177.546 82.931) (end 177.165 82.931) (width 0.25) (layer B.Cu) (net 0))
 (segment (start 177.165 82.931) (end 176.657 83.439) (width 0.25) (layer B.Cu) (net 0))
 (segment (start 176.657 83.439) (end 176.657 85.852) (width 0.25) (layer B.Cu) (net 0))
 (segment (start 176.149 86.36) (end 174.625 86.36) (width 0.25) (layer B.Cu) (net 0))
 (segment (start 176.657 85.852) (end 176.149 86.36) (width 0.25) (layer B.Cu) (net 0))
 (segment (start 176.01 82.435) (end 174.625 83.82) (width 0.25) (layer B.Cu) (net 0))
 (segment (start 177.755 82.435) (end 176.01 82.435) (width 0.25) (layer B.Cu) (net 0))
 (segment (start 174.67 81.235) (end 174.625 81.28) (width 0.25) (layer B.Cu) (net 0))
 (segment (start 178.955 81.235) (end 174.67 81.235) (width 0.25) (layer B.Cu) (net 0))
 (segment (start 179.455 81.235) (end 179.455 81.03) (width 0.25) (layer B.Cu) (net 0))
 (segment (start 179.455 81.03) (end 179.451 81.026) (width 0.25) (layer B.Cu) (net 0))
 (segment (start 179.451 81.026) (end 179.451 80.645) (width 0.25) (layer B.Cu) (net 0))
 (segment (start 179.451 80.645) (end 179.07 80.264) (width 0.25) (layer B.Cu) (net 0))
 (segment (start 179.07 80.264) (end 176.911 80.264) (width 0.25) (layer B.Cu) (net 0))
 (segment (start 176.911 80.264) (end 176.403 79.756) (width 0.25) (layer B.Cu) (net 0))
 (segment (start 176.403 79.756) (end 176.403 79.248) (width 0.25) (layer B.Cu) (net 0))
 (segment (start 175.895 78.74) (end 174.625 78.74) (width 0.25) (layer B.Cu) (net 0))
 (segment (start 176.403 79.248) (end 175.895 78.74) (width 0.25) (layer B.Cu) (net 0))
 (segment (start 179.955 81.235) (end 179.955 81.03) (width 0.25) (layer B.Cu) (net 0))
 (segment (start 179.955 81.03) (end 179.959 81.026) (width 0.25) (layer B.Cu) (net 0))
 (segment (start 179.959 81.026) (end 179.959 80.518) (width 0.25) (layer B.Cu) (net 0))
 (segment (start 179.959 80.518) (end 179.324 79.883) (width 0.25) (layer B.Cu) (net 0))
 (segment (start 179.324 79.883) (end 177.038 79.883) (width 0.25) (layer B.Cu) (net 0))
 (segment (start 177.038 79.883) (end 176.784 79.629) (width 0.25) (layer B.Cu) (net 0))
 (segment (start 176.784 79.629) (end 176.784 76.835) (width 0.25) (layer B.Cu) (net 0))
 (segment (start 176.149 76.2) (end 174.625 76.2) (width 0.25) (layer B.Cu) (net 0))
 (segment (start 176.784 76.835) (end 176.149 76.2) (width 0.25) (layer B.Cu) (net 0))
 (segment (start 180.455 81.235) (end 180.455 80.379) (width 0.25) (layer B.Cu) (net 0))
 (segment (start 180.455 80.379) (end 179.451 79.375) (width 0.25) (layer B.Cu) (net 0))
 (segment (start 179.451 79.375) (end 177.419 79.375) (width 0.25) (layer B.Cu) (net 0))
 (segment (start 177.419 79.375) (end 177.165 79.121) (width 0.25) (layer B.Cu) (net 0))
 (segment (start 177.165 79.121) (end 177.165 74.676) (width 0.25) (layer B.Cu) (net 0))
 (segment (start 176.149 73.66) (end 174.625 73.66) (width 0.25) (layer B.Cu) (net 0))
 (segment (start 177.165 74.676) (end 176.149 73.66) (width 0.25) (layer B.Cu) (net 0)))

